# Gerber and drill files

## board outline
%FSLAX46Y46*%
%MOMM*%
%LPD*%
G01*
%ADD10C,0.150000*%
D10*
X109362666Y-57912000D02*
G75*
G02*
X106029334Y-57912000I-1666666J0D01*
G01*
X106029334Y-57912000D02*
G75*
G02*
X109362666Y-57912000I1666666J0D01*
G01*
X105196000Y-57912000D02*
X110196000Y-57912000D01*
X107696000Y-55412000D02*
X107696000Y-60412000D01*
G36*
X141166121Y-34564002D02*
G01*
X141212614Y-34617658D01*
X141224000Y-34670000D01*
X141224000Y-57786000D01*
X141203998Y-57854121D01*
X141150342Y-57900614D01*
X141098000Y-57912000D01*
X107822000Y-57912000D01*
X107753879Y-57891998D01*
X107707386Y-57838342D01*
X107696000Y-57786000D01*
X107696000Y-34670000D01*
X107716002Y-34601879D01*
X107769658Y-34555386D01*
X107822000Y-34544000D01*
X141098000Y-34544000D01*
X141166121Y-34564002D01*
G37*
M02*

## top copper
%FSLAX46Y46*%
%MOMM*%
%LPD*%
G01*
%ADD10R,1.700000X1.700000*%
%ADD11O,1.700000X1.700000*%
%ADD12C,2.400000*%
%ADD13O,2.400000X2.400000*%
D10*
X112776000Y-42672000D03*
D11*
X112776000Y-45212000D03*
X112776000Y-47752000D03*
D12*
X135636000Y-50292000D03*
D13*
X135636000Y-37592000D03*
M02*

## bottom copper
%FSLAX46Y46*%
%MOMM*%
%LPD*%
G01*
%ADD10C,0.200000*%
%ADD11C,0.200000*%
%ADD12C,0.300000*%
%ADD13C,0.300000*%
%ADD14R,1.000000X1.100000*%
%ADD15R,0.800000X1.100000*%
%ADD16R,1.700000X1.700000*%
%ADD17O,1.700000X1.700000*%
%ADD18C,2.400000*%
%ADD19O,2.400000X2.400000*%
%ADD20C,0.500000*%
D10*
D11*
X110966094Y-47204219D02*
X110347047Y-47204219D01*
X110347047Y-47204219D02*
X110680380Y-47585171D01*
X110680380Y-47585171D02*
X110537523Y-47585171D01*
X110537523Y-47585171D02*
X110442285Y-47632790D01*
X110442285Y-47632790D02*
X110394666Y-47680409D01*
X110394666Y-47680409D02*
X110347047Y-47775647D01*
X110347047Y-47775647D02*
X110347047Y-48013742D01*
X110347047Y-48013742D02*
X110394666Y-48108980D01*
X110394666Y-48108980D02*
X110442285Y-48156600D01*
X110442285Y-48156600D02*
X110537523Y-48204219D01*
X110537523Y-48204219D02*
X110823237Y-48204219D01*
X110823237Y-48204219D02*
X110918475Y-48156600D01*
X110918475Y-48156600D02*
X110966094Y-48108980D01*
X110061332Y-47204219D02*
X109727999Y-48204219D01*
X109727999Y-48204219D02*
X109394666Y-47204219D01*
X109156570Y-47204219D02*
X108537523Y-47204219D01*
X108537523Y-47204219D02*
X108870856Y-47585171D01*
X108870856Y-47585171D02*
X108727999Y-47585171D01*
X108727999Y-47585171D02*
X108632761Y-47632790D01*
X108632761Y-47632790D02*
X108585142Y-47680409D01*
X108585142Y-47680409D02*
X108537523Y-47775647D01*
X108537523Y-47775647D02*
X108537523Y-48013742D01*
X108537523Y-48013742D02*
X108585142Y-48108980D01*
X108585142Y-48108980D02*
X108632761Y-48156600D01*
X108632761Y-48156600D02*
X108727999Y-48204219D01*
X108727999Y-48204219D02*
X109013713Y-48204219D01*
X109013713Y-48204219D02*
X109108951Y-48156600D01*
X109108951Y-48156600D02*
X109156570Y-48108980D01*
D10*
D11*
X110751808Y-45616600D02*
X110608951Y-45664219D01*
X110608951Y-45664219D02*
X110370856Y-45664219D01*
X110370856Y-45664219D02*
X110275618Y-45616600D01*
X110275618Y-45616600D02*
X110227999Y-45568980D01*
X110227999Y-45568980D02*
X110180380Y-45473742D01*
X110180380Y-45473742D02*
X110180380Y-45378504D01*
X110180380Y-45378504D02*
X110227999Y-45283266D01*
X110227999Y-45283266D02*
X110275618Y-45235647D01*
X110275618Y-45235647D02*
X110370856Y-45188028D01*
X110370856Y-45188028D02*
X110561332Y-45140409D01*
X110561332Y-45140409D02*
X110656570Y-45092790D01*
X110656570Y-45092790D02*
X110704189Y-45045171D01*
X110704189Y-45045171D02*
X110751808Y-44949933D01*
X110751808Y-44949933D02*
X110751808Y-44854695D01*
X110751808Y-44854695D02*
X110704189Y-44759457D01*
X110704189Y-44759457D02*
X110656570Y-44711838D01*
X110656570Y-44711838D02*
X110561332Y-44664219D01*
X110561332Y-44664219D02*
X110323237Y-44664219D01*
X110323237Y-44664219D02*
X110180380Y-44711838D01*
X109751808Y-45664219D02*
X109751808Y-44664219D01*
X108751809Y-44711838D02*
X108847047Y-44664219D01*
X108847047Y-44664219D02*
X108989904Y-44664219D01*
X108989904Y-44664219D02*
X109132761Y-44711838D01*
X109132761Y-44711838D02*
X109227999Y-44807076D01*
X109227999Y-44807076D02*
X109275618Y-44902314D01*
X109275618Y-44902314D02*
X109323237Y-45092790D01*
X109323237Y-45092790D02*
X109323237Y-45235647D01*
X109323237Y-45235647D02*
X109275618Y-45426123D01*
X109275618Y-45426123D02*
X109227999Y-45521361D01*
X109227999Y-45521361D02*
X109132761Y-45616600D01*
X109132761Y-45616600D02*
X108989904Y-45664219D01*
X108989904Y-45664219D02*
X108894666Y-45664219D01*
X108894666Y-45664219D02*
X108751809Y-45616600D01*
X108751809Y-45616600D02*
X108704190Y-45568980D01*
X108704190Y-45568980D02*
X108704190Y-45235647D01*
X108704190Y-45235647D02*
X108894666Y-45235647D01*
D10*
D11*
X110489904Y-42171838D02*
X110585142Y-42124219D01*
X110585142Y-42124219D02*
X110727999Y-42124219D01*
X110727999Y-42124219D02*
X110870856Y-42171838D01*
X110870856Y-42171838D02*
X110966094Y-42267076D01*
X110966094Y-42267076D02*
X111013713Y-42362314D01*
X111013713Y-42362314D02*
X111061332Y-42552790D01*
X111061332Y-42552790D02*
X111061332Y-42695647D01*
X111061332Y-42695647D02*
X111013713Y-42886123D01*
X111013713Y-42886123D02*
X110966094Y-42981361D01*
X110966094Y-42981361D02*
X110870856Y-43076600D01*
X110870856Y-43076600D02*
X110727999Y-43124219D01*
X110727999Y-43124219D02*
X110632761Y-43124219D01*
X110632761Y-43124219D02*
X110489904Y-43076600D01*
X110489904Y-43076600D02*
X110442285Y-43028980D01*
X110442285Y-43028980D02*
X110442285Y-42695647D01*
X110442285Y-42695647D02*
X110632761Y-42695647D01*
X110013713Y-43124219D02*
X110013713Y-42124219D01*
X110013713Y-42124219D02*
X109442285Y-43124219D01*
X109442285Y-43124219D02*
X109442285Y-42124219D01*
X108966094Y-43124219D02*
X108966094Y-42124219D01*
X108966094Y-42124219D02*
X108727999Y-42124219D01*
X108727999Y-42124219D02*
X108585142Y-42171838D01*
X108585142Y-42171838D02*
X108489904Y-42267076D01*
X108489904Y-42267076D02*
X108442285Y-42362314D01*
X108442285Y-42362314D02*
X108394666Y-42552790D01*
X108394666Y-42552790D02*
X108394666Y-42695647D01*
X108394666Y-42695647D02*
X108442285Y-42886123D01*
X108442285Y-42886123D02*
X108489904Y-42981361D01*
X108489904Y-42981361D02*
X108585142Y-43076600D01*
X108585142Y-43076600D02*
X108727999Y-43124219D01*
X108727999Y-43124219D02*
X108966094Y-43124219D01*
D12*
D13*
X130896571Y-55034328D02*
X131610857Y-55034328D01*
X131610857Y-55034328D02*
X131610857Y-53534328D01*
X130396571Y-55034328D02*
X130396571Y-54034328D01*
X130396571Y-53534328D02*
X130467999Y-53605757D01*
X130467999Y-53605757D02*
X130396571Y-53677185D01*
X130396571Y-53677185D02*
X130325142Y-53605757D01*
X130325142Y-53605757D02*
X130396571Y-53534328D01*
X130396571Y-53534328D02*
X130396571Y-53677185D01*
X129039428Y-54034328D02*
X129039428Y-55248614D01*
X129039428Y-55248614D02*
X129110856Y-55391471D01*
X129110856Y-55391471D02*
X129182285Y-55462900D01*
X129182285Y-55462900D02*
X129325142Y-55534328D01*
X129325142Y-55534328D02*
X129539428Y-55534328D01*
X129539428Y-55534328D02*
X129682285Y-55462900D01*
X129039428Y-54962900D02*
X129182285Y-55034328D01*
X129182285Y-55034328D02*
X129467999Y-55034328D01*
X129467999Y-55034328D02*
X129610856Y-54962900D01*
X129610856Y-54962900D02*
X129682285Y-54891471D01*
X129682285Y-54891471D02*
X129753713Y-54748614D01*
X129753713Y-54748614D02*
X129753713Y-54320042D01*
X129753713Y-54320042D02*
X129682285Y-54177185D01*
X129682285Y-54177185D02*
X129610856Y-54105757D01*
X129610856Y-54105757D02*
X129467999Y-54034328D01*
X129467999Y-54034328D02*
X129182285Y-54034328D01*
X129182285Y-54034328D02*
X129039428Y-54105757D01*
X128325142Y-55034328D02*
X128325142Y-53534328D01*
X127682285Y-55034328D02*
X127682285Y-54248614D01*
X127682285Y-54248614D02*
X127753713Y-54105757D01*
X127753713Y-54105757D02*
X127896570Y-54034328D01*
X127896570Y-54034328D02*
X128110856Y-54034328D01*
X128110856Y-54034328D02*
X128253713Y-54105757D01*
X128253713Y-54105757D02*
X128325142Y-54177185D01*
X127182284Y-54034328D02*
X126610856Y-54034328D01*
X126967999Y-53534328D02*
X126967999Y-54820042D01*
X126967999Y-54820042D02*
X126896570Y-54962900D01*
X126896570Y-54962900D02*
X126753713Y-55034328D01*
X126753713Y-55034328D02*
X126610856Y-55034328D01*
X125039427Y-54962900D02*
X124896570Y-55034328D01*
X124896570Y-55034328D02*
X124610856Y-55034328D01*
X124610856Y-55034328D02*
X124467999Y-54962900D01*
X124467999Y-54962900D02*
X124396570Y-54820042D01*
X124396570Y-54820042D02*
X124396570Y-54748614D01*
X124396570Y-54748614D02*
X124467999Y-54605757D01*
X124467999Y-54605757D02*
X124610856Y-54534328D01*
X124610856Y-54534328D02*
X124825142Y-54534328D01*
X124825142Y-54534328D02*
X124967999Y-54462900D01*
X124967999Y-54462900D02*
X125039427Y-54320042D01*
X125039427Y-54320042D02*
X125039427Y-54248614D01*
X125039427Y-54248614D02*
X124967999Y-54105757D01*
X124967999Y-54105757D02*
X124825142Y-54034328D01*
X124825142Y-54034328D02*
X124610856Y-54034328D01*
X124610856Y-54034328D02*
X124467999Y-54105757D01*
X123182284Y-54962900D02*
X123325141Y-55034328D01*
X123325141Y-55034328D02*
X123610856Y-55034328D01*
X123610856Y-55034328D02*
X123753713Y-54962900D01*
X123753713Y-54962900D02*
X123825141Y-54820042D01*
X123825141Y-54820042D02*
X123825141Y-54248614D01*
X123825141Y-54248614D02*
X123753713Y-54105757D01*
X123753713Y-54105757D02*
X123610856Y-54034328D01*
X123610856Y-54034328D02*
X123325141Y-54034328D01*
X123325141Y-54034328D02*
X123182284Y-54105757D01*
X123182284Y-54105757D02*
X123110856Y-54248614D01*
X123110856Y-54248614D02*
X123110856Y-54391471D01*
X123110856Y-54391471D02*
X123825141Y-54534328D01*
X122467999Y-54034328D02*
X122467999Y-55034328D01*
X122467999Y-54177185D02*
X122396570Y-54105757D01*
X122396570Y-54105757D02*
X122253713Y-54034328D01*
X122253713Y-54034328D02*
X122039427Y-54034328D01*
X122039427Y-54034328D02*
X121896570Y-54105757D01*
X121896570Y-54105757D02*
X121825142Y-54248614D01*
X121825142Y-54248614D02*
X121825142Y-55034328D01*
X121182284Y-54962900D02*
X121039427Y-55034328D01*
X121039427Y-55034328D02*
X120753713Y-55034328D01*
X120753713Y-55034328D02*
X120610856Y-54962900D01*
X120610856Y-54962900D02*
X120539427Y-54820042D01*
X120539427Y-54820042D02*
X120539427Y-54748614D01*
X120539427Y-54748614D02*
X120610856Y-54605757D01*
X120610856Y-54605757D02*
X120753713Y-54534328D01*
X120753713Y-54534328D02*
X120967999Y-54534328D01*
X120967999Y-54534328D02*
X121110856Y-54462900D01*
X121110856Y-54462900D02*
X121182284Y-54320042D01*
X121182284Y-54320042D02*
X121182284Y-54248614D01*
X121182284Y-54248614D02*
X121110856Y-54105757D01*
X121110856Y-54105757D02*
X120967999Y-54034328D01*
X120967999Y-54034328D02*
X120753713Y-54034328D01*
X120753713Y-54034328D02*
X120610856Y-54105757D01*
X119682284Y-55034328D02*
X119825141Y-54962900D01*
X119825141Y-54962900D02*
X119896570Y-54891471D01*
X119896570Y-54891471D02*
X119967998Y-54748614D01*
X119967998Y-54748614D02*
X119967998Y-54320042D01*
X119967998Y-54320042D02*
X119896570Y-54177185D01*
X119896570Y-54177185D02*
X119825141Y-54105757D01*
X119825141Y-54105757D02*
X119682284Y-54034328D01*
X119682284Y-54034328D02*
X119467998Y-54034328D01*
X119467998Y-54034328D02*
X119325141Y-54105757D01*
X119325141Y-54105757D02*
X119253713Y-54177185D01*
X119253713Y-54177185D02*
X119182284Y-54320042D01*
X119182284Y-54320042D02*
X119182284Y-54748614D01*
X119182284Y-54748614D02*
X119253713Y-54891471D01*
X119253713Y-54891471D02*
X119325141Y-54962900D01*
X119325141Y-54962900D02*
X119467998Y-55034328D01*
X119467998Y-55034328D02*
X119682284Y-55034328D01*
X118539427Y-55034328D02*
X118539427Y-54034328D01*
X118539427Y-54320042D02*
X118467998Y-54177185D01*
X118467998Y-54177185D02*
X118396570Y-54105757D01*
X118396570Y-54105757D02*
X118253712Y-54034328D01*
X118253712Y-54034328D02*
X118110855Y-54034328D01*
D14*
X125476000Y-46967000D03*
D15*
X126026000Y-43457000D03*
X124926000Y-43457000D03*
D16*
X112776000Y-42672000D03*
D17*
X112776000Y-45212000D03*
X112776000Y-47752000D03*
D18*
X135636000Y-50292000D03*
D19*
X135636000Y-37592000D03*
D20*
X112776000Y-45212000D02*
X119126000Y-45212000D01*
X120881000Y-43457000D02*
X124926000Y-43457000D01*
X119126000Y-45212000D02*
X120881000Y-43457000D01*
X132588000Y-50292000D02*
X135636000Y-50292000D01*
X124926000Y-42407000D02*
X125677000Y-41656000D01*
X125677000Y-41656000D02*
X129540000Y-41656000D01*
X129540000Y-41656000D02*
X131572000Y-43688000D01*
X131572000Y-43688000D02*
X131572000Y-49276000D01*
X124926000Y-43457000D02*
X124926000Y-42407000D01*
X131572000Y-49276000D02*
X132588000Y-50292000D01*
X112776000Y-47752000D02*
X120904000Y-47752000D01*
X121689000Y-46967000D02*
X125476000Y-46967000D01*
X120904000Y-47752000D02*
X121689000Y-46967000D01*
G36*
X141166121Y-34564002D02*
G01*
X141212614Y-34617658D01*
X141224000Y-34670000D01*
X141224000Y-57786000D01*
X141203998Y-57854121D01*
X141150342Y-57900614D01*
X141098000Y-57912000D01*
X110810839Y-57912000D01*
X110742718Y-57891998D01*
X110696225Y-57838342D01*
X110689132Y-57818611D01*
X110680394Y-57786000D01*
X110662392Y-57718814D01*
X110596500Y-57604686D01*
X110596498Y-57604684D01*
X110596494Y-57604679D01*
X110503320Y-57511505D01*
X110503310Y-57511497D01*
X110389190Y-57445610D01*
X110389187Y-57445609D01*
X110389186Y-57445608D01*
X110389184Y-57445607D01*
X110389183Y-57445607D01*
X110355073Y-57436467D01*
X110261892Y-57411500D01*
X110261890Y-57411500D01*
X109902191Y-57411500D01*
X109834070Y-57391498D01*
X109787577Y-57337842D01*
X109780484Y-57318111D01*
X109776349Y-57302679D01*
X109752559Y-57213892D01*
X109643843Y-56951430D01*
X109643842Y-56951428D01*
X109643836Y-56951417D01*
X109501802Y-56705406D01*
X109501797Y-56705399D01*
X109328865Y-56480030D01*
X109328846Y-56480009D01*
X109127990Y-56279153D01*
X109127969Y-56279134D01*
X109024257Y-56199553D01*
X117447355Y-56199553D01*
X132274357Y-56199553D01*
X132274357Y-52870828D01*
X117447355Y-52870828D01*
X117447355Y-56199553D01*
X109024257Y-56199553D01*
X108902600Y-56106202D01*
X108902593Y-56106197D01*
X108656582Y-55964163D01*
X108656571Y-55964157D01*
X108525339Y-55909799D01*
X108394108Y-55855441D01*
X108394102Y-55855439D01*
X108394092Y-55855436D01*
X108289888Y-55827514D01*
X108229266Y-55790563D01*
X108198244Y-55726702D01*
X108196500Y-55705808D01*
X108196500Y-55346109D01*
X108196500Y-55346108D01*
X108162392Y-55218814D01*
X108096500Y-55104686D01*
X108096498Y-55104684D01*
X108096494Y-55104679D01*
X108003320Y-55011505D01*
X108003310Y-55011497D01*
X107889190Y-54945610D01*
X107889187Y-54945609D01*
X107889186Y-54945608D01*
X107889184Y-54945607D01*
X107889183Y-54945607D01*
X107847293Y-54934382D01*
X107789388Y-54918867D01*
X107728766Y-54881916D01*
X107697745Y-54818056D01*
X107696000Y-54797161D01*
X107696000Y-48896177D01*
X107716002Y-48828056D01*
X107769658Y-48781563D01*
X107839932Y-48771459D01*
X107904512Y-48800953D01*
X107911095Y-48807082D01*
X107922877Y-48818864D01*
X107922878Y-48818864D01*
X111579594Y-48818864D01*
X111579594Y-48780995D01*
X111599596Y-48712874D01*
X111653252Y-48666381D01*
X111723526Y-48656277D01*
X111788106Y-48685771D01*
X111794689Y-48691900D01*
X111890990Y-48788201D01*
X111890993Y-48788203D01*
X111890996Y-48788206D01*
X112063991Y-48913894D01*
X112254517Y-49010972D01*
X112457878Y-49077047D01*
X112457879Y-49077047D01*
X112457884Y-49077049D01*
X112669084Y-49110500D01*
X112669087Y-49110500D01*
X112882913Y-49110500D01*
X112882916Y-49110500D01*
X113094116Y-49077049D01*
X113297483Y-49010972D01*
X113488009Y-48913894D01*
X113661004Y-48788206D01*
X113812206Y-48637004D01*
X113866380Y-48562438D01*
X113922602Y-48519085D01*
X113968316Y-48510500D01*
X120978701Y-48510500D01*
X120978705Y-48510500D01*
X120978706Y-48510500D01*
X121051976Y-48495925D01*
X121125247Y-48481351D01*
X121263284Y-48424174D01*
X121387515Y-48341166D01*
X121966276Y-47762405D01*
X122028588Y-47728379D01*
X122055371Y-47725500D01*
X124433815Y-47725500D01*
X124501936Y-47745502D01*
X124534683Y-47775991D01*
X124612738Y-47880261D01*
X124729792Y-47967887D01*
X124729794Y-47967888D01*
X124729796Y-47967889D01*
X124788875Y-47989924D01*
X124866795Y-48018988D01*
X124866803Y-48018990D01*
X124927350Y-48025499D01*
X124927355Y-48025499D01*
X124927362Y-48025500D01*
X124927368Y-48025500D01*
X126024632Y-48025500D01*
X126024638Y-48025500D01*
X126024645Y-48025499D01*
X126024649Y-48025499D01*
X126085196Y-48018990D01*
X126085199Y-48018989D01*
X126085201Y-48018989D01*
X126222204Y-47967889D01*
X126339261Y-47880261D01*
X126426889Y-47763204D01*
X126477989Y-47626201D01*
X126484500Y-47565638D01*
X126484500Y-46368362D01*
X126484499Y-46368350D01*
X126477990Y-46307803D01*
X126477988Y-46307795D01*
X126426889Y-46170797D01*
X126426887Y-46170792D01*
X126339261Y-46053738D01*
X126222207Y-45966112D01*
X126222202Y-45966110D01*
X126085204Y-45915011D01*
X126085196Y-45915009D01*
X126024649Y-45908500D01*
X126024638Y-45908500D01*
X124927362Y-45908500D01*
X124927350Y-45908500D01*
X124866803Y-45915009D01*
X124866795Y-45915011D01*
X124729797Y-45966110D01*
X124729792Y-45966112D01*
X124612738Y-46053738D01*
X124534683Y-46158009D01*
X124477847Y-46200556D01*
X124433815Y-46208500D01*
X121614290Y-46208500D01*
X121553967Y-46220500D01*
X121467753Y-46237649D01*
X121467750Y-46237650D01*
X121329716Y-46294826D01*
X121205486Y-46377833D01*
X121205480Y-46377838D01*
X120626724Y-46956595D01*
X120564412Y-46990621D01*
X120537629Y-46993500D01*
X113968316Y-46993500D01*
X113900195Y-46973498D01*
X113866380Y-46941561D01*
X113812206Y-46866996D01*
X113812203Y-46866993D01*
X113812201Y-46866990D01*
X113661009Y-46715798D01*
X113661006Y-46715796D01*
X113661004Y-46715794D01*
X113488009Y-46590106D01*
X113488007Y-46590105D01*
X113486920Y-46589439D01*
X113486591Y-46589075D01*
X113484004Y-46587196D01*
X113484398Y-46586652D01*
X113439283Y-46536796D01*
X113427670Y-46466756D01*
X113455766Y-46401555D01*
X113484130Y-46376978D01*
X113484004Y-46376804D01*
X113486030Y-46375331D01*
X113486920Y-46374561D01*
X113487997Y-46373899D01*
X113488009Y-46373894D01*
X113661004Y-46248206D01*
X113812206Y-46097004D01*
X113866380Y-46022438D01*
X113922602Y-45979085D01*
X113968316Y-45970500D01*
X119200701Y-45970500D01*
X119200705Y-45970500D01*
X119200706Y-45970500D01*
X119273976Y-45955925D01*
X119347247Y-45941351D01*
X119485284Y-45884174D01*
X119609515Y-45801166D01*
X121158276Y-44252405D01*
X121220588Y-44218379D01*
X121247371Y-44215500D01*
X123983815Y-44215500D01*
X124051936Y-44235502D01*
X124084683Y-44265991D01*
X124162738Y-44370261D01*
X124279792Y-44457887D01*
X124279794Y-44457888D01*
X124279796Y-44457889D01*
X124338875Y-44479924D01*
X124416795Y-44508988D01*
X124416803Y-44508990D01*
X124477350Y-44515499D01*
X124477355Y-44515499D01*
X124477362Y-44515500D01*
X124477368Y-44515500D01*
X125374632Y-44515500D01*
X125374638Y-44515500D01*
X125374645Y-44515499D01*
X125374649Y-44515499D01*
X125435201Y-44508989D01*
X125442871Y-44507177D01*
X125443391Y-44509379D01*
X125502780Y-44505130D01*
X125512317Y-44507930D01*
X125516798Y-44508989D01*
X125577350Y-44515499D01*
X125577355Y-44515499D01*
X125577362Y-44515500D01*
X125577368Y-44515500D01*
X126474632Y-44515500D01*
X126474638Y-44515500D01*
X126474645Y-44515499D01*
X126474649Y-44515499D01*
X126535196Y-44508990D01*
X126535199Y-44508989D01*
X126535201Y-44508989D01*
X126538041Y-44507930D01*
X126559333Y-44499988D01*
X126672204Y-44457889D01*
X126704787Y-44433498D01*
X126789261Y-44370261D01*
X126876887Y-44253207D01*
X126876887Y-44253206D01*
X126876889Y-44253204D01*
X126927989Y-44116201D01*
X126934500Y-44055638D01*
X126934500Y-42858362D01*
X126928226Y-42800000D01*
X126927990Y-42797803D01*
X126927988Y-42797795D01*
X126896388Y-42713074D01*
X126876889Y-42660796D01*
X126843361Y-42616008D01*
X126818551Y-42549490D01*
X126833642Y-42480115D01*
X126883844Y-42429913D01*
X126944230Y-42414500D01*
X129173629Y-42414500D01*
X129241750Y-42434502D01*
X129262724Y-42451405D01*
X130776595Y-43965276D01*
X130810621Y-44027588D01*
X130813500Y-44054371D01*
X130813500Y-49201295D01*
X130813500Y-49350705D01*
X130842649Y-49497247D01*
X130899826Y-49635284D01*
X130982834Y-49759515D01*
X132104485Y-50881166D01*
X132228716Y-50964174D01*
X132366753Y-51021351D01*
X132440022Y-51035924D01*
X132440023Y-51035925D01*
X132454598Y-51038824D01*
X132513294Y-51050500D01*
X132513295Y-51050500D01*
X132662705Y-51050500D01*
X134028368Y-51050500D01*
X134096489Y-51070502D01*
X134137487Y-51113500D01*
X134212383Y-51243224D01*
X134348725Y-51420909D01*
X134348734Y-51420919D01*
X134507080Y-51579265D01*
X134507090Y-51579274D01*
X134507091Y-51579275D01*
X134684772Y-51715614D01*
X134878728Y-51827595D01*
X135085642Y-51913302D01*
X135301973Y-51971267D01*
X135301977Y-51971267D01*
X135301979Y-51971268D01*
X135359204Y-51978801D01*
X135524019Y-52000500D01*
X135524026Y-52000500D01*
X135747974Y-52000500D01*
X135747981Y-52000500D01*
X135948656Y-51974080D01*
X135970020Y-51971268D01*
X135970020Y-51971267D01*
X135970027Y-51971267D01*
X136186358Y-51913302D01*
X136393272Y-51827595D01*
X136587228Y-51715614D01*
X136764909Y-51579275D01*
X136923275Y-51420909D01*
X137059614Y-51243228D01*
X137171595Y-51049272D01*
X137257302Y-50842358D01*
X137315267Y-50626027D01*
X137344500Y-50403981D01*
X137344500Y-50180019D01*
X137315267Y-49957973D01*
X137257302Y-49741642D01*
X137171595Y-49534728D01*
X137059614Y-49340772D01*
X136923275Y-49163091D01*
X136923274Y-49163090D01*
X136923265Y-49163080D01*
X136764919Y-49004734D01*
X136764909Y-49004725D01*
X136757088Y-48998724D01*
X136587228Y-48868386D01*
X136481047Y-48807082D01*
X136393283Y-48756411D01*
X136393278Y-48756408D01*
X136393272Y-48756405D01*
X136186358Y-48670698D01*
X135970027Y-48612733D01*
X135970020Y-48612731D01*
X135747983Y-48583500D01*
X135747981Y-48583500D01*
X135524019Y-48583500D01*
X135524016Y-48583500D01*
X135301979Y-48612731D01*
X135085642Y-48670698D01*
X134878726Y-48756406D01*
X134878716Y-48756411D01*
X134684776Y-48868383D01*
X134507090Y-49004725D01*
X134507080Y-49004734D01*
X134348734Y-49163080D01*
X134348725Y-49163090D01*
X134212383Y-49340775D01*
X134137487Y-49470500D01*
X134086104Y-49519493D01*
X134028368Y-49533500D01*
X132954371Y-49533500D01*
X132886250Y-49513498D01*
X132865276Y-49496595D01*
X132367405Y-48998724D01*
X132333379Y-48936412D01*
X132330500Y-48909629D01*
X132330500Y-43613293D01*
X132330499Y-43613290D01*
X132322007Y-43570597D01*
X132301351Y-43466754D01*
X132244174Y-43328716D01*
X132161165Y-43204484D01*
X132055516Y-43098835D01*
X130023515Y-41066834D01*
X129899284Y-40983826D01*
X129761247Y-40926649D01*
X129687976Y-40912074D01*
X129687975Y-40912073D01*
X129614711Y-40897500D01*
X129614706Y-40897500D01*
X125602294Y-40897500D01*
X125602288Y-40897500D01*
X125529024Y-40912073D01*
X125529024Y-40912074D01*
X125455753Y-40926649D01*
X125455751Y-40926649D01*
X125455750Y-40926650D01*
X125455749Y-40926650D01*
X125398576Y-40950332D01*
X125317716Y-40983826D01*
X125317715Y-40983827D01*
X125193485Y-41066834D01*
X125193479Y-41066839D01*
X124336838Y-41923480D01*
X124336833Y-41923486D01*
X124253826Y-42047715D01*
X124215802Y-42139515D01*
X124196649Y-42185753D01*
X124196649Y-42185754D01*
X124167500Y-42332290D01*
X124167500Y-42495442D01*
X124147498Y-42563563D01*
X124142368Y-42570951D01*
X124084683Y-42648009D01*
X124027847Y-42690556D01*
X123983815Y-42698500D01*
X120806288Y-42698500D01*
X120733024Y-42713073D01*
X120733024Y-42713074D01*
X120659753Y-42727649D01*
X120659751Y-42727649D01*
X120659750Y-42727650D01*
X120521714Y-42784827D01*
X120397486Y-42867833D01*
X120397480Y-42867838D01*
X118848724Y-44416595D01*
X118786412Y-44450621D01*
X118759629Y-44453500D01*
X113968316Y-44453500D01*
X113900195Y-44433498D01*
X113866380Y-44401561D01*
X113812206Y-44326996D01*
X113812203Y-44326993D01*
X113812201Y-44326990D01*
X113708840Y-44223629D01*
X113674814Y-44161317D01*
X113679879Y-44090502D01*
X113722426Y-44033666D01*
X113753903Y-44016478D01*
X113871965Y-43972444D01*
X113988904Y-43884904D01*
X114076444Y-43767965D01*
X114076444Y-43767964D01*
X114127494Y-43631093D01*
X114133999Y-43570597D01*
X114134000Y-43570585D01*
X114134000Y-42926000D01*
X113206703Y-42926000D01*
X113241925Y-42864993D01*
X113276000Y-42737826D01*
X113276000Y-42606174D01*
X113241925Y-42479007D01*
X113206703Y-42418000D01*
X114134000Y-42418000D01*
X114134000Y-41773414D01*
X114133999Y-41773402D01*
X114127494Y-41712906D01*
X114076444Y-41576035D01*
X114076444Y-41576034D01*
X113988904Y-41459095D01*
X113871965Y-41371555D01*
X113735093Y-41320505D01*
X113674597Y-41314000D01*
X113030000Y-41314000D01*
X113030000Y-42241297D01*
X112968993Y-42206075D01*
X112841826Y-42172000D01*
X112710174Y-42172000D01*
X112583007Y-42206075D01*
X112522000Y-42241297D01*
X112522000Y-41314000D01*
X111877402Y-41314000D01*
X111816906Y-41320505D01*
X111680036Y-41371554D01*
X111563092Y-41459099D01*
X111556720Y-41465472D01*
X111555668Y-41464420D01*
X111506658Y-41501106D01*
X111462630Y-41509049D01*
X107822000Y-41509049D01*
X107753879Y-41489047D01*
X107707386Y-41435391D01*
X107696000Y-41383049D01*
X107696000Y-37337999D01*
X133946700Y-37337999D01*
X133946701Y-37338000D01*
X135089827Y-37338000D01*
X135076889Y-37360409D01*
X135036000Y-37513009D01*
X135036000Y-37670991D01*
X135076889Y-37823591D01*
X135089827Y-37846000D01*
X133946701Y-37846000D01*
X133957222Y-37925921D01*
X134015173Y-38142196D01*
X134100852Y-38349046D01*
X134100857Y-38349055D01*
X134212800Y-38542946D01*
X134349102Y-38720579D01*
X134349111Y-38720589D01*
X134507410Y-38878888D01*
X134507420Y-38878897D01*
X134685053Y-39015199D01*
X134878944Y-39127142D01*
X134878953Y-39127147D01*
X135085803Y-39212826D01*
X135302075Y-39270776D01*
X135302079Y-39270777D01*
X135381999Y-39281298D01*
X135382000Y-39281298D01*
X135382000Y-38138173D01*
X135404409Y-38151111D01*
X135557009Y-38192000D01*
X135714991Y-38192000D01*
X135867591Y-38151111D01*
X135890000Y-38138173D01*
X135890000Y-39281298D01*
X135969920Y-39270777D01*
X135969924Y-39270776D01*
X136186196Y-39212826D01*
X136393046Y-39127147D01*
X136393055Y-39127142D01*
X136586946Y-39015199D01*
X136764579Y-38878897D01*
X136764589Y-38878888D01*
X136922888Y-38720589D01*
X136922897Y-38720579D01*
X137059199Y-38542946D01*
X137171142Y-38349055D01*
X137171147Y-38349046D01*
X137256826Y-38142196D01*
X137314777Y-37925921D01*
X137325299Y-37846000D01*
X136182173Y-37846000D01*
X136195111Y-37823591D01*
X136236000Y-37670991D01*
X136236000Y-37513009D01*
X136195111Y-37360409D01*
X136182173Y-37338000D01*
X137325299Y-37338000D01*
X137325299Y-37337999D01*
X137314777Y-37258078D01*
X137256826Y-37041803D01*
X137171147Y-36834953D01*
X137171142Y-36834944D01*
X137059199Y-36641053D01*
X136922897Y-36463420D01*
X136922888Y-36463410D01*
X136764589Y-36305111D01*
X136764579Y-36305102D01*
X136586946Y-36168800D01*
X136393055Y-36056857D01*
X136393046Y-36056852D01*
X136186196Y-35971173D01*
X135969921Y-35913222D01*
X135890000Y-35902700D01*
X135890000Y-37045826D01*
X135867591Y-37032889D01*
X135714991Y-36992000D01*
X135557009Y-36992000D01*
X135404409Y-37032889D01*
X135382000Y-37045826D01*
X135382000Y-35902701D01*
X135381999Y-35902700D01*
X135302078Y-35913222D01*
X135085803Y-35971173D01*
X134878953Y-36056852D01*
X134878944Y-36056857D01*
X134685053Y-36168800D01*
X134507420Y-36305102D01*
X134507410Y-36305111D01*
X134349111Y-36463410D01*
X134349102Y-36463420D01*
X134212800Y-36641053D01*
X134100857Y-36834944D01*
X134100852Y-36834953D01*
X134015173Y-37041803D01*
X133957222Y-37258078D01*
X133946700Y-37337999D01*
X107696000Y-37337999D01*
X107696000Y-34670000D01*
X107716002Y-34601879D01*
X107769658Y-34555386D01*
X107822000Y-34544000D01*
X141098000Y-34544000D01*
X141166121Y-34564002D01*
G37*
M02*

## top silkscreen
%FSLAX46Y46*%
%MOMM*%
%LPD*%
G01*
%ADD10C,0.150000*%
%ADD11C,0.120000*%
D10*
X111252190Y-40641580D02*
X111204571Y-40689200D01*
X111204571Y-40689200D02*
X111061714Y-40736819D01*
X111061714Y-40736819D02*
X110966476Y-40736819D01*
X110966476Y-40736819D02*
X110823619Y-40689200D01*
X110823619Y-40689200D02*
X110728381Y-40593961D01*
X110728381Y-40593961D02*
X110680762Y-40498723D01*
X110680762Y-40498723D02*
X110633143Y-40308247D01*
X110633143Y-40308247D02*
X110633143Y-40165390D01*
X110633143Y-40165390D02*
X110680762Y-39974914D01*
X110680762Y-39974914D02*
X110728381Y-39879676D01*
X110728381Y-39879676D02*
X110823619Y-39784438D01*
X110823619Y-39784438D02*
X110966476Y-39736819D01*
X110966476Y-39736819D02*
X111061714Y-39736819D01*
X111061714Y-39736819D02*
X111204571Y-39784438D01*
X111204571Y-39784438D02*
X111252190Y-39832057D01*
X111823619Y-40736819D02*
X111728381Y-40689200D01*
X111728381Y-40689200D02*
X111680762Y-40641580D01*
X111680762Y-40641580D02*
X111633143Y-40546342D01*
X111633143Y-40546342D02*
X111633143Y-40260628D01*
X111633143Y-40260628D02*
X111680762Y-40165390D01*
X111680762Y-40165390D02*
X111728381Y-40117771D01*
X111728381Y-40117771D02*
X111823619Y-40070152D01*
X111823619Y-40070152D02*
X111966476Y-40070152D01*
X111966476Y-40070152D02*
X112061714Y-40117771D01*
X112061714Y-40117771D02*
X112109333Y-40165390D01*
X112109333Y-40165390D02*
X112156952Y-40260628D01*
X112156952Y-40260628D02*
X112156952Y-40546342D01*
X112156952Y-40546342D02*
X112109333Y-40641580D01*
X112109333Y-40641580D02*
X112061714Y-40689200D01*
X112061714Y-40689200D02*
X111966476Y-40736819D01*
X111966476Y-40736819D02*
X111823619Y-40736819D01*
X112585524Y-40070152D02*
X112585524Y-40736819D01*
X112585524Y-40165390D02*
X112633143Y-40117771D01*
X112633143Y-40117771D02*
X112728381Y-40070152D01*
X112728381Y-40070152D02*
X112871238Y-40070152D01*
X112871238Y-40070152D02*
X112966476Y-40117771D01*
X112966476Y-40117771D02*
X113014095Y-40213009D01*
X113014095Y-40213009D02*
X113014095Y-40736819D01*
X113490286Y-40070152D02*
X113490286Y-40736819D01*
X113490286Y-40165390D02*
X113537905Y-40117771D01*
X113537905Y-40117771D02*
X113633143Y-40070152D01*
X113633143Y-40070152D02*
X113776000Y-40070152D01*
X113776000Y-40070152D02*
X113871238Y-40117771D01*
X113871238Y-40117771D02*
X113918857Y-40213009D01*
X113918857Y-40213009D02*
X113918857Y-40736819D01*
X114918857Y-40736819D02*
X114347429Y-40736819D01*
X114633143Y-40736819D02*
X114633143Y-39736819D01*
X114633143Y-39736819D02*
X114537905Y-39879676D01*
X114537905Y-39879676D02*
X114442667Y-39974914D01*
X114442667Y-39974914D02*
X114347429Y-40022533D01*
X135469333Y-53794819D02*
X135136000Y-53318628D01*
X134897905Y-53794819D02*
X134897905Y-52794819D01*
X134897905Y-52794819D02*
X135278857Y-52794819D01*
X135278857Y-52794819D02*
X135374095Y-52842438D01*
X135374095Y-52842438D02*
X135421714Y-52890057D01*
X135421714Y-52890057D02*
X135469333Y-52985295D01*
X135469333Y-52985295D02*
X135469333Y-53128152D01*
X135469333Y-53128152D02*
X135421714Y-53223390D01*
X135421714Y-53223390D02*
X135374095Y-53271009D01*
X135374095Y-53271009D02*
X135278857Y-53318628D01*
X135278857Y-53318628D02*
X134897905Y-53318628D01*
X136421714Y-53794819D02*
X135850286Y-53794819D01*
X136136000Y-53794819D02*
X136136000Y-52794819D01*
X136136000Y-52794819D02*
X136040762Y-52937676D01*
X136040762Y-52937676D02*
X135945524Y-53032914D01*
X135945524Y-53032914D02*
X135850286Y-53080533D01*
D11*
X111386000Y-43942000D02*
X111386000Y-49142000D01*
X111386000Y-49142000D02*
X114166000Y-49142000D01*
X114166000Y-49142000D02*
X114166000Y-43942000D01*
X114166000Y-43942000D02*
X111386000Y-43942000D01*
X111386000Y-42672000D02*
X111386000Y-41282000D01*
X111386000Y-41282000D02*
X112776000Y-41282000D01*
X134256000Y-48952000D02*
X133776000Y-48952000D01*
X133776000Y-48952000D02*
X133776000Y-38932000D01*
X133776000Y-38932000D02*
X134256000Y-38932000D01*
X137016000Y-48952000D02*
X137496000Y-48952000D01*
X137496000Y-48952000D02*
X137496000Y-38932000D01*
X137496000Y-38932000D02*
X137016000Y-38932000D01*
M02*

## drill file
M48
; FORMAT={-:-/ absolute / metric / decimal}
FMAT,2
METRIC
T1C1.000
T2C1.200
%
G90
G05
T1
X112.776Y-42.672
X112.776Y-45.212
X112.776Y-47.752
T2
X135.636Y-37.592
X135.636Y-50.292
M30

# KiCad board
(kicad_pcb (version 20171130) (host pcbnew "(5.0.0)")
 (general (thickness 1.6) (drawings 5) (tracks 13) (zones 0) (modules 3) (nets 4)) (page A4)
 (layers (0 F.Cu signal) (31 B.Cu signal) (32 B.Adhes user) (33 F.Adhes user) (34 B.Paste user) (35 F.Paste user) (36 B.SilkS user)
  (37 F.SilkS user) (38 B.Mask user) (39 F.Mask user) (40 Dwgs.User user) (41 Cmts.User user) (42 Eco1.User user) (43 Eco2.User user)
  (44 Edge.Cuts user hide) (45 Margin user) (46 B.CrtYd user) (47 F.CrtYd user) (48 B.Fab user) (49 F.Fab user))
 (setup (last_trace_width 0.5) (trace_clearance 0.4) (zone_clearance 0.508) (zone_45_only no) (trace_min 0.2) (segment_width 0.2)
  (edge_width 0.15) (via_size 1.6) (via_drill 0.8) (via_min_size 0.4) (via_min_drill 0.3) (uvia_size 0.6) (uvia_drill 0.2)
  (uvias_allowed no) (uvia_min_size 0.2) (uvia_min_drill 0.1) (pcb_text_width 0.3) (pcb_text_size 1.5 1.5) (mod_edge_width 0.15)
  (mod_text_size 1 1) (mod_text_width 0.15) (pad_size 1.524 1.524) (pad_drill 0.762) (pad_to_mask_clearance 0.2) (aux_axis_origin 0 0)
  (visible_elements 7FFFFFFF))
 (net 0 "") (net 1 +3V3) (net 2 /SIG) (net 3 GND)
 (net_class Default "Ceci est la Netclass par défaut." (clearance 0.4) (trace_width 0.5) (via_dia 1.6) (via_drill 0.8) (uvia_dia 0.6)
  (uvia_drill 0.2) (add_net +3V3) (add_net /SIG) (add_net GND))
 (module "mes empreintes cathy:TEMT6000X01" (layer B.Cu) (at 125.476 45.212 270)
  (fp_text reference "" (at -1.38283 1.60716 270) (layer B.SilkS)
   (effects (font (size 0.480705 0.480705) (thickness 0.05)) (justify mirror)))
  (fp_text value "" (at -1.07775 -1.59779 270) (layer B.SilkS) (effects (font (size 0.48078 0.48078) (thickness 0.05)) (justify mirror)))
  (pad 3 smd rect (at 1.755 0 270) (size 1.1 1) (layers B.Cu B.Paste B.Mask) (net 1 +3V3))
  (pad 2 smd rect (at -1.755 -0.55 270) (size 1.1 0.8) (layers B.Cu B.Paste B.Mask))
  (pad 1 smd rect (at -1.755 0.55 270) (size 1.1 0.8) (layers B.Cu B.Paste B.Mask) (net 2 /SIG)))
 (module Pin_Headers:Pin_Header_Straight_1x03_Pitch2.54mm (layer F.Cu) (at 112.776 42.672)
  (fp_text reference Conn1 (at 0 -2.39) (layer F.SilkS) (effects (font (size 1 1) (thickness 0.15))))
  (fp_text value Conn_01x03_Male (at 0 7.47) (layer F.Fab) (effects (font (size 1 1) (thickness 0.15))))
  (fp_line (start -1.39 1.27) (end -1.39 6.47) (layer F.SilkS) (width 0.12))
  (fp_line (start -1.39 6.47) (end 1.39 6.47) (layer F.SilkS) (width 0.12))
  (fp_line (start 1.39 6.47) (end 1.39 1.27) (layer F.SilkS) (width 0.12))
  (fp_line (start 1.39 1.27) (end -1.39 1.27) (layer F.SilkS) (width 0.12))
  (fp_line (start -1.39 0) (end -1.39 -1.39) (layer F.SilkS) (width 0.12))
  (fp_line (start -1.39 -1.39) (end 0 -1.39) (layer F.SilkS) (width 0.12))
  (pad 1 thru_hole rect (at 0 0) (size 1.7 1.7) (drill 1) (layers *.Cu *.Mask) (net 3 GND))
  (pad 2 thru_hole oval (at 0 2.54) (size 1.7 1.7) (drill 1) (layers *.Cu *.Mask) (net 2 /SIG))
  (pad 3 thru_hole oval (at 0 5.08) (size 1.7 1.7) (drill 1) (layers *.Cu *.Mask) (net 1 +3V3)))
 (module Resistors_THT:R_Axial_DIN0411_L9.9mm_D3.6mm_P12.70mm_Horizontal (layer F.Cu) (at 135.636 50.292 90)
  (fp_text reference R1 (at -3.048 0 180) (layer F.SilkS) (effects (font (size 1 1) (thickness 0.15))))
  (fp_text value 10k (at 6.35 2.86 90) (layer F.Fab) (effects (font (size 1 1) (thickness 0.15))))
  (fp_line (start 1.34 -1.38) (end 1.34 -1.86) (layer F.SilkS) (width 0.12))
  (fp_line (start 1.34 -1.86) (end 11.36 -1.86) (layer F.SilkS) (width 0.12))
  (fp_line (start 11.36 -1.86) (end 11.36 -1.38) (layer F.SilkS) (width 0.12))
  (fp_line (start 1.34 1.38) (end 1.34 1.86) (layer F.SilkS) (width 0.12))
  (fp_line (start 1.34 1.86) (end 11.36 1.86) (layer F.SilkS) (width 0.12))
  (fp_line (start 11.36 1.86) (end 11.36 1.38) (layer F.SilkS) (width 0.12))
  (pad 1 thru_hole circle (at 0 0 90) (size 2.4 2.4) (drill 1.2) (layers *.Cu *.Mask) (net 2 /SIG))
  (pad 2 thru_hole oval (at 12.7 0 90) (size 2.4 2.4) (drill 1.2) (layers *.Cu *.Mask) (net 3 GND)))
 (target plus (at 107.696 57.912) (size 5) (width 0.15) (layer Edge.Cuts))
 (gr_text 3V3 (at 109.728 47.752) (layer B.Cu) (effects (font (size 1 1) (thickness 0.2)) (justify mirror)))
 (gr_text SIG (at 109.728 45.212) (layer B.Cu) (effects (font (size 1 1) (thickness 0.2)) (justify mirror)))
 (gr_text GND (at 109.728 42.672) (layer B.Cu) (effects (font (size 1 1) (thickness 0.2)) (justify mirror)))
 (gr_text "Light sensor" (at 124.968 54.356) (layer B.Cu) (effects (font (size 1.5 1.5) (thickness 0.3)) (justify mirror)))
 (segment (start 112.776 45.212) (end 119.126 45.212) (width 0.5) (layer B.Cu) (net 2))
 (segment (start 120.881 43.457) (end 124.926 43.457) (width 0.5) (layer B.Cu) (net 2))
 (segment (start 119.126 45.212) (end 120.881 43.457) (width 0.5) (layer B.Cu) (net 2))
 (segment (start 132.588 50.292) (end 135.636 50.292) (width 0.5) (layer B.Cu) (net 2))
 (segment (start 124.926 42.407) (end 125.677 41.656) (width 0.5) (layer B.Cu) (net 2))
 (segment (start 125.677 41.656) (end 129.54 41.656) (width 0.5) (layer B.Cu) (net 2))
 (segment (start 129.54 41.656) (end 131.572 43.688) (width 0.5) (layer B.Cu) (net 2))
 (segment (start 131.572 43.688) (end 131.572 49.276) (width 0.5) (layer B.Cu) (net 2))
 (segment (start 124.926 43.457) (end 124.926 42.407) (width 0.5) (layer B.Cu) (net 2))
 (segment (start 131.572 49.276) (end 132.588 50.292) (width 0.5) (layer B.Cu) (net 2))
 (segment (start 112.776 47.752) (end 120.904 47.752) (width 0.5) (layer B.Cu) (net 1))
 (segment (start 121.689 46.967) (end 125.476 46.967) (width 0.5) (layer B.Cu) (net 1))
 (segment (start 120.904 47.752) (end 121.689 46.967) (width 0.5) (layer B.Cu) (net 1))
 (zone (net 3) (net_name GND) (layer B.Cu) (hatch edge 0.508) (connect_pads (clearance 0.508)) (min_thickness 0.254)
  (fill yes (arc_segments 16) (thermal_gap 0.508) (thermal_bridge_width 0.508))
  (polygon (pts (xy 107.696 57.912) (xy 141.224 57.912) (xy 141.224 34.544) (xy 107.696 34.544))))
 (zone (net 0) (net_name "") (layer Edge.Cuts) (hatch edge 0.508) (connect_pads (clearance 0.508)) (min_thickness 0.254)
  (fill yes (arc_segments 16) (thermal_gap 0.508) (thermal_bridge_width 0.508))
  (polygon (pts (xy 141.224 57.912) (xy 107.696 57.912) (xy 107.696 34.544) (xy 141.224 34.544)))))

